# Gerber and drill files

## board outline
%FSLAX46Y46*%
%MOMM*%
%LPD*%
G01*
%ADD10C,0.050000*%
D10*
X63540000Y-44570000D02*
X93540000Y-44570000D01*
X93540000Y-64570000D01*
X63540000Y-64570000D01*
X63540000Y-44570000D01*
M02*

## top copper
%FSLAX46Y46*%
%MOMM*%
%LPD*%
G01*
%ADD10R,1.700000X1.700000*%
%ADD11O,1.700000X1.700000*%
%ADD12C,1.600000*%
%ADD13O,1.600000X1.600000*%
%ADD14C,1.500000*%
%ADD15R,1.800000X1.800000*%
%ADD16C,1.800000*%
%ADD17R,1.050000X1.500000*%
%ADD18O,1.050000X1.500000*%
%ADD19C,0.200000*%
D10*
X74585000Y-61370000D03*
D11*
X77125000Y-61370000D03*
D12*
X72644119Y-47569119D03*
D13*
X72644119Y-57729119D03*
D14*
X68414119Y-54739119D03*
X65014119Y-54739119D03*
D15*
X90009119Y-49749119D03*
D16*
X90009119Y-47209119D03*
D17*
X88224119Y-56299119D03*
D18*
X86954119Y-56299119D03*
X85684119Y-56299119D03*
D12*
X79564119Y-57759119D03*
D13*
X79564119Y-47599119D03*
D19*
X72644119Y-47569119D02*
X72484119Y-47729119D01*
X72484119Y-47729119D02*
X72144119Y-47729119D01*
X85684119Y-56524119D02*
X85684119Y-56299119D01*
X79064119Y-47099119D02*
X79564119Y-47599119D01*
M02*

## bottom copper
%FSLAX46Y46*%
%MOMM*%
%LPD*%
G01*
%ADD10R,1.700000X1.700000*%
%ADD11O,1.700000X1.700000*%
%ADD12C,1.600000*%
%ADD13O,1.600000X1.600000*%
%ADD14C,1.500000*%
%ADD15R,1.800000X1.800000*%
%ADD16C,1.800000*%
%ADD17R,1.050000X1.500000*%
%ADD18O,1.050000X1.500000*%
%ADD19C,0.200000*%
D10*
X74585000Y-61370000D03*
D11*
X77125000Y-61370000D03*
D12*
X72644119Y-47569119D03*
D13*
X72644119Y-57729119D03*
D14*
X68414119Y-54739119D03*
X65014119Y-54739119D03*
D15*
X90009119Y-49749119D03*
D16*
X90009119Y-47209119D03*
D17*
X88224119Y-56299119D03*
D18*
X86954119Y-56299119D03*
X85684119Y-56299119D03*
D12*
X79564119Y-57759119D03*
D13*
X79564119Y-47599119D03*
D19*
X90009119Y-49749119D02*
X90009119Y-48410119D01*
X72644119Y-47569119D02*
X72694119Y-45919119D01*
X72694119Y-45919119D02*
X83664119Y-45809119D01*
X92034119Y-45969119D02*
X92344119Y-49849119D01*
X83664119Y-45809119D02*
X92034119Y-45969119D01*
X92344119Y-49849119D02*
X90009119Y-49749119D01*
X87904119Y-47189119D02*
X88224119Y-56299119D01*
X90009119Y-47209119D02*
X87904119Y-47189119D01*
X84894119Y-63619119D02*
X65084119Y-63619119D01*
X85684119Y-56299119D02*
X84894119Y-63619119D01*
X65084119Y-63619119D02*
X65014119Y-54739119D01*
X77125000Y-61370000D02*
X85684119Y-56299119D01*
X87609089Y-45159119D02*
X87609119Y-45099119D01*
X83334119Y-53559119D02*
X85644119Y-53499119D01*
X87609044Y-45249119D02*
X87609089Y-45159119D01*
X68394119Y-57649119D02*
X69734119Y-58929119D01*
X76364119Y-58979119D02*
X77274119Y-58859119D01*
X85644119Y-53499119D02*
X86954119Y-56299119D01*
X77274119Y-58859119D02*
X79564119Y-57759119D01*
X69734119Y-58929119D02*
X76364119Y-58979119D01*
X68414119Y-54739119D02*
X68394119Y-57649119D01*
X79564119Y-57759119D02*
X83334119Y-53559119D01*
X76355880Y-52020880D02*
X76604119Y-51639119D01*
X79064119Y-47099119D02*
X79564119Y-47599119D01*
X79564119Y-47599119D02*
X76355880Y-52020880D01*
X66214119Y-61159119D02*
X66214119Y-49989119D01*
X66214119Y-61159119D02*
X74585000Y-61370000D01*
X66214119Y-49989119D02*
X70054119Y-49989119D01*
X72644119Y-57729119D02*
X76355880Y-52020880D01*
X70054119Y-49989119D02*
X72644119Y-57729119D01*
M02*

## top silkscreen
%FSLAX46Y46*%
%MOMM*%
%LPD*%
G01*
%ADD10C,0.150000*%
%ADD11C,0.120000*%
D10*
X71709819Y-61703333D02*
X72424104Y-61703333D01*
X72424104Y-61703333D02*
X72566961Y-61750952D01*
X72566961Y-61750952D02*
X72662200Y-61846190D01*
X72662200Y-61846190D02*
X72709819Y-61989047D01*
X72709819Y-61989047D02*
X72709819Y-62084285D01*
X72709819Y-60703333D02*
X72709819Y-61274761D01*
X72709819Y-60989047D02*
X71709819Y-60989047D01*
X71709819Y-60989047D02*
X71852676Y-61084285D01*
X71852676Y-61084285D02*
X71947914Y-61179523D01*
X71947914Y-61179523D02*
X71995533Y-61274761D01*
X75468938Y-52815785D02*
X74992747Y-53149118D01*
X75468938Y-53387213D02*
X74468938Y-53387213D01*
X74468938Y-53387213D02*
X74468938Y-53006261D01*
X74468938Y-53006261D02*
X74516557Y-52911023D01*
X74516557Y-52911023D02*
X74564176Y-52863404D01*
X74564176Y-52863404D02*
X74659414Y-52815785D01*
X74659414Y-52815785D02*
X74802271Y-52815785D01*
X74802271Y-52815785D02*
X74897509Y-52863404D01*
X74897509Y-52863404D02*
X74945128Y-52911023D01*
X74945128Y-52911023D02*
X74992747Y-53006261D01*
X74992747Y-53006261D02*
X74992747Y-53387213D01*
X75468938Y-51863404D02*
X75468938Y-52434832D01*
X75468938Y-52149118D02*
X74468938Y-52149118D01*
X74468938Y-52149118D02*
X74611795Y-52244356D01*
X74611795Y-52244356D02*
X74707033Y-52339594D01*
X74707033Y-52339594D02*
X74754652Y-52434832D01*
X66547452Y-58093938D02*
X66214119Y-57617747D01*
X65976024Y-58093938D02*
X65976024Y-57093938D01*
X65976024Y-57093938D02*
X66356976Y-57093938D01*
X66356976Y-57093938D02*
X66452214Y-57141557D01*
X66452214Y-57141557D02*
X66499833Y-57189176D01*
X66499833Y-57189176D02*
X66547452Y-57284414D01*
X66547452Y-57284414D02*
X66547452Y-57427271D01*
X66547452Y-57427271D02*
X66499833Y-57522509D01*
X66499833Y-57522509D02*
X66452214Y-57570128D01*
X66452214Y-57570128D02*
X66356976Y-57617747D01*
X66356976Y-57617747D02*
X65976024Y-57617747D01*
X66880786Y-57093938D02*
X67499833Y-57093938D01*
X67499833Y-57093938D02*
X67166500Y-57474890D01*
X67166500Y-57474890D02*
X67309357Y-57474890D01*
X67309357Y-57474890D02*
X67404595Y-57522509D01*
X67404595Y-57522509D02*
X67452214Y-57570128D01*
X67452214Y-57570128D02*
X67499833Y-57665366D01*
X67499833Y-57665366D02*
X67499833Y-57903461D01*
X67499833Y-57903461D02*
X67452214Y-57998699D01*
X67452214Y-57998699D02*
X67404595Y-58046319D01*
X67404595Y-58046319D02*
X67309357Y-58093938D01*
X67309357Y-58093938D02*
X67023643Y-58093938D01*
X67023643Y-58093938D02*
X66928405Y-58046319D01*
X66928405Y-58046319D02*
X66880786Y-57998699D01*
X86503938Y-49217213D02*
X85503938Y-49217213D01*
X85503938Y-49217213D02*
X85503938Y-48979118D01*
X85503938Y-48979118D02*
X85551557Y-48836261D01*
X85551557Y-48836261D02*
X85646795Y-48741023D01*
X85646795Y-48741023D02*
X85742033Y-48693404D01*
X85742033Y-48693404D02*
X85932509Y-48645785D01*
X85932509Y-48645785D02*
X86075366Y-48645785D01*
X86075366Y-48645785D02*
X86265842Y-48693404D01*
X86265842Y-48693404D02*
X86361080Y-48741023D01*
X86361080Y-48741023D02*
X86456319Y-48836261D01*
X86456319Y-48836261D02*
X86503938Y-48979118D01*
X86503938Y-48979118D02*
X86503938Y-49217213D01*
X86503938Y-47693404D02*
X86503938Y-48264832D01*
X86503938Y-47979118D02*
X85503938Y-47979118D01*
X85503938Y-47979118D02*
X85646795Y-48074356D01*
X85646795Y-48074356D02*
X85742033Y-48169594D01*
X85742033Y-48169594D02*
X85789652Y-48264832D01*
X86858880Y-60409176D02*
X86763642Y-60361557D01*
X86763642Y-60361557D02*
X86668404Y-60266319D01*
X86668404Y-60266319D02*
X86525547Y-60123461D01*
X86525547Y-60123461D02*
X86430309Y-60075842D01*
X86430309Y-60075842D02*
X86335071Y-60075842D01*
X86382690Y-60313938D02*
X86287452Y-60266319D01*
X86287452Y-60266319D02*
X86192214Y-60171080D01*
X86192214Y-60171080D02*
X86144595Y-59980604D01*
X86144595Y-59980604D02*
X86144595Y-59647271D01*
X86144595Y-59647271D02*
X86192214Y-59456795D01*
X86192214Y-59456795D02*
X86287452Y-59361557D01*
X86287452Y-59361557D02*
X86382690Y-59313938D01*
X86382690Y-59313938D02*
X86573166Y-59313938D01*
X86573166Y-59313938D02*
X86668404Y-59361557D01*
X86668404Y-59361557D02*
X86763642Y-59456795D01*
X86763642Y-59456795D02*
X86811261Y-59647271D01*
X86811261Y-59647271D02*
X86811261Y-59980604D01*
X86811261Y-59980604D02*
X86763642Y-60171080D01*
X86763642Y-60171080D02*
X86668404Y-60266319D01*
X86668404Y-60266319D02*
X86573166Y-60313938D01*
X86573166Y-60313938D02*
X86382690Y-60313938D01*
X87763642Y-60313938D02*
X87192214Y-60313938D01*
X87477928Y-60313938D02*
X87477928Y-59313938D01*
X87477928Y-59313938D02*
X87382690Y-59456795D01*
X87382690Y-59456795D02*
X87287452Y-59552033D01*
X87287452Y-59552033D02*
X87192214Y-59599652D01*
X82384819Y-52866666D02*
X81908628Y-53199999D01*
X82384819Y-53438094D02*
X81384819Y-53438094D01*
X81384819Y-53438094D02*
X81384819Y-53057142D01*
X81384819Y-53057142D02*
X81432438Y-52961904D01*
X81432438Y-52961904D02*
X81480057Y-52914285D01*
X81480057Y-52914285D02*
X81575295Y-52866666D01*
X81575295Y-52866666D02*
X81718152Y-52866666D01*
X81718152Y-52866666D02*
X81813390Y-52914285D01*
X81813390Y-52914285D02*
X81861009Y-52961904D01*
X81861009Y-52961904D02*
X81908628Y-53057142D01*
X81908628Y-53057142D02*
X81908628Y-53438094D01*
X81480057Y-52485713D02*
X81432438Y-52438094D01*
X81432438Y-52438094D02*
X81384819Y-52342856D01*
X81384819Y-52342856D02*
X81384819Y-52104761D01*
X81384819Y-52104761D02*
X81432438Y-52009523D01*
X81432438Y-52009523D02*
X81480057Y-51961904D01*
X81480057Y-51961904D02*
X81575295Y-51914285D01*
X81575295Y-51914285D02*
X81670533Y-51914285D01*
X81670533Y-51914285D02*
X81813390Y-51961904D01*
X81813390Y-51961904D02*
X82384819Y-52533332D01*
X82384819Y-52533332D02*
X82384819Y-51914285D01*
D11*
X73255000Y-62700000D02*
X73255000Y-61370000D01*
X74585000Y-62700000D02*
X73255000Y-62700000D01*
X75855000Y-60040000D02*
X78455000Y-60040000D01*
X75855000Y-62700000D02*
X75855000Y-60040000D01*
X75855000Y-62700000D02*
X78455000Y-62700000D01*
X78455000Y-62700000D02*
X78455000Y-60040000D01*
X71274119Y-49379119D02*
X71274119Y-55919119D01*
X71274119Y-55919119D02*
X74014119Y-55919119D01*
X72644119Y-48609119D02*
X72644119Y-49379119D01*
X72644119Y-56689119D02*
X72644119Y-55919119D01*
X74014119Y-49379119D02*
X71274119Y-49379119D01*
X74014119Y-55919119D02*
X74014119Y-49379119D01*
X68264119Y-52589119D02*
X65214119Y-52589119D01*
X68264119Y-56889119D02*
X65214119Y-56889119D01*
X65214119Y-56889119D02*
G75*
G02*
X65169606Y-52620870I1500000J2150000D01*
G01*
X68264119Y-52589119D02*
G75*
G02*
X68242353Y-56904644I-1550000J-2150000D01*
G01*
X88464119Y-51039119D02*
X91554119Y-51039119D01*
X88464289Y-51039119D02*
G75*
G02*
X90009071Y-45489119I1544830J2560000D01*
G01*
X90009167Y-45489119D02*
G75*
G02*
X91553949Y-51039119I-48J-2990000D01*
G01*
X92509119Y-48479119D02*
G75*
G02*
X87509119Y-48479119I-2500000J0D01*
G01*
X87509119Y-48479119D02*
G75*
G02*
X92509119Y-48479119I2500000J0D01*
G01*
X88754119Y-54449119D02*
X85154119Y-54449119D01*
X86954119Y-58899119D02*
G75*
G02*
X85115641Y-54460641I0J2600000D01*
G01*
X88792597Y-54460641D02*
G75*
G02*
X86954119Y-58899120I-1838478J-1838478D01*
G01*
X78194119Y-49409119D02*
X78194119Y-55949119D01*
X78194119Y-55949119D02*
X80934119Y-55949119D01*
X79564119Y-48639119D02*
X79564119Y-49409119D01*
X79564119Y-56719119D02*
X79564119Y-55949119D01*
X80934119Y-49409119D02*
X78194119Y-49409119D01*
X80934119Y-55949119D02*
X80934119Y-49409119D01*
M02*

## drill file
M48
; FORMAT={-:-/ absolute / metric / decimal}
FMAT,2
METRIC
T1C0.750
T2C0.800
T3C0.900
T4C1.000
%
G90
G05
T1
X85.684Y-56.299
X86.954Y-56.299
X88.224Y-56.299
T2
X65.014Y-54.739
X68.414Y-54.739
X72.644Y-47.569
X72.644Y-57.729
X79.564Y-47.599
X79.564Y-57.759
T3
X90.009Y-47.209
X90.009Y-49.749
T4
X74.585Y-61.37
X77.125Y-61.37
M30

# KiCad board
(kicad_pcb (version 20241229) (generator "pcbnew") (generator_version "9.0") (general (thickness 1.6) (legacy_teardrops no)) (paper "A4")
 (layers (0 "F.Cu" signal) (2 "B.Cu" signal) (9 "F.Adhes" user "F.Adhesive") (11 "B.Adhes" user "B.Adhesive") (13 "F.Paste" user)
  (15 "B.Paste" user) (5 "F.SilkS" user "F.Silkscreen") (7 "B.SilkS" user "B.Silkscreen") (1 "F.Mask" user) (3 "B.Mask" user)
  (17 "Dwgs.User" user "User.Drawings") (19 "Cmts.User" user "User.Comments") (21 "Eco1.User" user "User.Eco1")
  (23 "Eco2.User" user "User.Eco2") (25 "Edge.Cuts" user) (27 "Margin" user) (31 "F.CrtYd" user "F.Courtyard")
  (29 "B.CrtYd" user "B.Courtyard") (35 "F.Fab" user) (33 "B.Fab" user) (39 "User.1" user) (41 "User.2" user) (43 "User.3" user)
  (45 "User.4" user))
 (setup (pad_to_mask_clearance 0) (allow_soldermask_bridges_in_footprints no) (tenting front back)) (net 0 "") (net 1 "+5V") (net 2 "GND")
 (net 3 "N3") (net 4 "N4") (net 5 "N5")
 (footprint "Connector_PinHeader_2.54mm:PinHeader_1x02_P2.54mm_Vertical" (layer "F.Cu") (at 74.585 61.37 90)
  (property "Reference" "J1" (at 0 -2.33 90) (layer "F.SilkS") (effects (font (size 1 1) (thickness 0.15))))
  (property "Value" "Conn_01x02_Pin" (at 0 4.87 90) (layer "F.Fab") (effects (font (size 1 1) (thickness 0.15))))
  (fp_line (start -1.33 -1.33) (end 0 -1.33) (stroke (width 0.12) (type solid)) (layer "F.SilkS"))
  (fp_line (start -1.33 0) (end -1.33 -1.33) (stroke (width 0.12) (type solid)) (layer "F.SilkS"))
  (fp_line (start 1.33 1.27) (end 1.33 3.87) (stroke (width 0.12) (type solid)) (layer "F.SilkS"))
  (fp_line (start -1.33 1.27) (end 1.33 1.27) (stroke (width 0.12) (type solid)) (layer "F.SilkS"))
  (fp_line (start -1.33 1.27) (end -1.33 3.87) (stroke (width 0.12) (type solid)) (layer "F.SilkS"))
  (fp_line (start -1.33 3.87) (end 1.33 3.87) (stroke (width 0.12) (type solid)) (layer "F.SilkS"))
  (pad "1" thru_hole rect (at 0 0 90) (size 1.7 1.7) (drill 1) (layers "*.Cu" "*.Mask") (remove_unused_layers no) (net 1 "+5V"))
  (pad "2" thru_hole oval (at 0 2.54 90) (size 1.7 1.7) (drill 1) (layers "*.Cu" "*.Mask") (remove_unused_layers no) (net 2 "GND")))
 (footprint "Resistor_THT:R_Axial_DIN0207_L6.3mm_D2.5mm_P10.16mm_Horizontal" (layer "F.Cu") (at 72.644119 47.569119 -90)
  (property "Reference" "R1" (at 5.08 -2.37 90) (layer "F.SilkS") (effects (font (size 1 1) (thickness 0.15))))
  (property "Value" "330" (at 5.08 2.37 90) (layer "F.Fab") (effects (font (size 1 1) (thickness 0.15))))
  (fp_line (start 1.81 1.37) (end 8.35 1.37) (stroke (width 0.12) (type solid)) (layer "F.SilkS"))
  (fp_line (start 8.35 1.37) (end 8.35 -1.37) (stroke (width 0.12) (type solid)) (layer "F.SilkS"))
  (fp_line (start 1.04 0) (end 1.81 0) (stroke (width 0.12) (type solid)) (layer "F.SilkS"))
  (fp_line (start 9.12 0) (end 8.35 0) (stroke (width 0.12) (type solid)) (layer "F.SilkS"))
  (fp_line (start 1.81 -1.37) (end 1.81 1.37) (stroke (width 0.12) (type solid)) (layer "F.SilkS"))
  (fp_line (start 8.35 -1.37) (end 1.81 -1.37) (stroke (width 0.12) (type solid)) (layer "F.SilkS"))
  (pad "1" thru_hole circle (at 0 0 270) (size 1.6 1.6) (drill 0.8) (layers "*.Cu" "*.Mask") (remove_unused_layers no) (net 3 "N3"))
  (pad "2" thru_hole oval (at 10.16 0 270) (size 1.6 1.6) (drill 0.8) (layers "*.Cu" "*.Mask") (remove_unused_layers no) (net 1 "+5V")))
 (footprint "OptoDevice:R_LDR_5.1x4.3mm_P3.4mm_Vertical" (layer "F.Cu") (at 68.414119 54.739119 180)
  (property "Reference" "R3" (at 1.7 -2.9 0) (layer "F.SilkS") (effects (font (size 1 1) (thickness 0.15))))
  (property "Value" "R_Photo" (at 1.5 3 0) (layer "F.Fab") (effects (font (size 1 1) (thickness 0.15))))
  (fp_line (start 0.15 2.15) (end 3.2 2.15) (stroke (width 0.12) (type solid)) (layer "F.SilkS"))
  (fp_line (start 0.15 -2.15) (end 3.2 -2.15) (stroke (width 0.12) (type solid)) (layer "F.SilkS"))
  (fp_arc (start 3.2 -2.15) (mid 4.321403 -0.027338) (end 3.244513 2.118249) (stroke (width 0.12) (type solid)) (layer "F.SilkS"))
  (fp_arc (start 0.15 2.15) (mid -0.950438 -0.013368) (end 0.171766 -2.165525) (stroke (width 0.12) (type solid)) (layer "F.SilkS"))
  (pad "1" thru_hole circle (at 0 0 180) (size 1.5 1.5) (drill 0.8) (layers "*.Cu" "*.Mask") (remove_unused_layers no) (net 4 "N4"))
  (pad "2" thru_hole circle (at 3.4 0 180) (size 1.5 1.5) (drill 0.8) (layers "*.Cu" "*.Mask") (remove_unused_layers no) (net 2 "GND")))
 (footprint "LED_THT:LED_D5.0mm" (layer "F.Cu") (at 90.009119 49.749119 90)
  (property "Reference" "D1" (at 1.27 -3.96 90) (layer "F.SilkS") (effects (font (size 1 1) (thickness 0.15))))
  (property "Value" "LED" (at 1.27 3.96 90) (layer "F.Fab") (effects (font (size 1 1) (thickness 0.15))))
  (fp_line (start -1.29 -1.545) (end -1.29 1.545) (stroke (width 0.12) (type solid)) (layer "F.SilkS"))
  (fp_arc (start -1.29 -1.54483) (mid 2.071756 -2.880501) (end 4.26 -0.000048) (stroke (width 0.12) (type solid)) (layer "F.SilkS"))
  (fp_arc (start 4.26 0.000048) (mid 2.071756 2.880501) (end -1.29 1.54483) (stroke (width 0.12) (type solid)) (layer "F.SilkS"))
  (fp_circle (center 1.27 0) (end 3.77 0) (stroke (width 0.12) (type solid)) (fill no) (layer "F.SilkS"))
  (pad "1" thru_hole rect (at 0 0 90) (size 1.8 1.8) (drill 0.9) (layers "*.Cu" "*.Mask") (remove_unused_layers no) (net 3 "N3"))
  (pad "2" thru_hole circle (at 2.54 0 90) (size 1.8 1.8) (drill 0.9) (layers "*.Cu" "*.Mask") (remove_unused_layers no) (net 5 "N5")))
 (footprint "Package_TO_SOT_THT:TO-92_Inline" (layer "F.Cu") (at 88.224119 56.299119 180)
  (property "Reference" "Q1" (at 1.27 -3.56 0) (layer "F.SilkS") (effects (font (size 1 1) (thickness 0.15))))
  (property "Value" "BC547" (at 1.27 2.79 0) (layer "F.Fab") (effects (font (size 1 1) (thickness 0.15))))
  (fp_line (start -0.53 1.85) (end 3.07 1.85) (stroke (width 0.12) (type solid)) (layer "F.SilkS"))
  (fp_arc (start 1.27 -2.6) (mid 3.672087 -0.994977) (end 3.108478 1.838478) (stroke (width 0.12) (type solid)) (layer "F.SilkS"))
  (fp_arc (start -0.568478 1.838478) (mid -1.132087 -0.994977) (end 1.27 -2.6) (stroke (width 0.12) (type solid)) (layer "F.SilkS"))
  (pad "1" thru_hole rect (at 0 0 180) (size 1.05 1.5) (drill 0.75) (layers "*.Cu" "*.Mask") (remove_unused_layers no) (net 5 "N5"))
  (pad "2" thru_hole oval (at 1.27 0 180) (size 1.05 1.5) (drill 0.75) (layers "*.Cu" "*.Mask") (remove_unused_layers no) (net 4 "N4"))
  (pad "3" thru_hole oval (at 2.54 0 180) (size 1.05 1.5) (drill 0.75) (layers "*.Cu" "*.Mask") (remove_unused_layers no) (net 2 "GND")))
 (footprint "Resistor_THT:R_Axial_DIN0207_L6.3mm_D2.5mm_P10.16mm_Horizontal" (layer "F.Cu") (at 79.564119 57.759119 90)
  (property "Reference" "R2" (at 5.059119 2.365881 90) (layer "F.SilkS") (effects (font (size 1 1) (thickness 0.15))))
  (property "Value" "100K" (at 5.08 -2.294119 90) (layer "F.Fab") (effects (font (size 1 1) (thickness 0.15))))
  (fp_line (start 8.35 -1.37) (end 1.81 -1.37) (stroke (width 0.12) (type solid)) (layer "F.SilkS"))
  (fp_line (start 1.81 -1.37) (end 1.81 1.37) (stroke (width 0.12) (type solid)) (layer "F.SilkS"))
  (fp_line (start 9.12 0) (end 8.35 0) (stroke (width 0.12) (type solid)) (layer "F.SilkS"))
  (fp_line (start 1.04 0) (end 1.81 0) (stroke (width 0.12) (type solid)) (layer "F.SilkS"))
  (fp_line (start 8.35 1.37) (end 8.35 -1.37) (stroke (width 0.12) (type solid)) (layer "F.SilkS"))
  (fp_line (start 1.81 1.37) (end 8.35 1.37) (stroke (width 0.12) (type solid)) (layer "F.SilkS"))
  (pad "1" thru_hole circle (at 0 0 90) (size 1.6 1.6) (drill 0.8) (layers "*.Cu" "*.Mask") (remove_unused_layers no) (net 4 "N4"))
  (pad "2" thru_hole oval (at 10.16 0 90) (size 1.6 1.6) (drill 0.8) (layers "*.Cu" "*.Mask") (remove_unused_layers no) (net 1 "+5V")))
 (gr_rect (start 93.54 64.57) (end 63.54 44.57) (stroke (width 0.05) (type solid)) (fill no) (layer "Edge.Cuts"))
 (segment (start 72.644119 47.569119) (end 72.484119 47.729119) (width 0.2) (layer "F.Cu") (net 3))
 (segment (start 72.484119 47.729119) (end 72.144119 47.729119) (width 0.2) (layer "F.Cu") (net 3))
 (segment (start 90.009119 49.749119) (end 90.009119 48.410119) (width 0.2) (layer "B.Cu") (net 3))
 (segment (start 72.644119 47.569119) (end 72.694119 45.919119) (width 0.2) (layer "B.Cu") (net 3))
 (segment (start 72.694119 45.919119) (end 83.664119 45.809119) (width 0.2) (layer "B.Cu") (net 3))
 (segment (start 92.034119 45.969119) (end 92.344119 49.849119) (width 0.2) (layer "B.Cu") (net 3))
 (segment (start 83.664119 45.809119) (end 92.034119 45.969119) (width 0.2) (layer "B.Cu") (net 3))
 (segment (start 92.344119 49.849119) (end 90.009119 49.749119) (width 0.2) (layer "B.Cu") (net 3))
 (segment (start 87.904119 47.189119) (end 88.224119 56.299119) (width 0.2) (layer "B.Cu") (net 5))
 (segment (start 90.009119 47.209119) (end 87.904119 47.189119) (width 0.2) (layer "B.Cu") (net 5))
 (segment (start 85.684119 56.524119) (end 85.684119 56.299119) (width 0.2) (layer "F.Cu") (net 2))
 (segment (start 84.894119 63.619119) (end 65.084119 63.619119) (width 0.2) (layer "B.Cu") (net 2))
 (segment (start 85.684119 56.299119) (end 84.894119 63.619119) (width 0.2) (layer "B.Cu") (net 2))
 (segment (start 65.084119 63.619119) (end 65.014119 54.739119) (width 0.2) (layer "B.Cu") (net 2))
 (segment (start 77.125 61.37) (end 85.684119 56.299119) (width 0.2) (layer "B.Cu") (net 2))
 (segment (start 87.609089 45.159119) (end 87.609119 45.099119) (width 0.2) (layer "B.Cu") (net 4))
 (segment (start 83.334119 53.559119) (end 85.644119 53.499119) (width 0.2) (layer "B.Cu") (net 4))
 (segment (start 87.609044 45.249119) (end 87.609089 45.159119) (width 0.2) (layer "B.Cu") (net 4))
 (segment (start 68.394119 57.649119) (end 69.734119 58.929119) (width 0.2) (layer "B.Cu") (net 4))
 (segment (start 76.364119 58.979119) (end 77.274119 58.859119) (width 0.2) (layer "B.Cu") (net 4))
 (segment (start 85.644119 53.499119) (end 86.954119 56.299119) (width 0.2) (layer "B.Cu") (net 4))
 (segment (start 77.274119 58.859119) (end 79.564119 57.759119) (width 0.2) (layer "B.Cu") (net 4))
 (segment (start 69.734119 58.929119) (end 76.364119 58.979119) (width 0.2) (layer "B.Cu") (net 4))
 (segment (start 68.414119 54.739119) (end 68.394119 57.649119) (width 0.2) (layer "B.Cu") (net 4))
 (segment (start 79.564119 57.759119) (end 83.334119 53.559119) (width 0.2) (layer "B.Cu") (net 4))
 (segment (start 79.064119 47.099119) (end 79.564119 47.599119) (width 0.2) (layer "F.Cu") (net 1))
 (segment (start 76.35588 52.02088) (end 76.604119 51.639119) (width 0.2) (layer "B.Cu") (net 1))
 (segment (start 79.064119 47.099119) (end 79.564119 47.599119) (width 0.2) (layer "B.Cu") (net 1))
 (segment (start 79.564119 47.599119) (end 76.35588 52.02088) (width 0.2) (layer "B.Cu") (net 1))
 (segment (start 66.214119 61.159119) (end 66.214119 49.989119) (width 0.2) (layer "B.Cu") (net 1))
 (segment (start 66.214119 61.159119) (end 74.585 61.37) (width 0.2) (layer "B.Cu") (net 1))
 (segment (start 66.214119 49.989119) (end 70.054119 49.989119) (width 0.2) (layer "B.Cu") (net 1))
 (segment (start 72.644119 57.729119) (end 76.35588 52.02088) (width 0.2) (layer "B.Cu") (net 1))
 (segment (start 70.054119 49.989119) (end 72.644119 57.729119) (width 0.2) (layer "B.Cu") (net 1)))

